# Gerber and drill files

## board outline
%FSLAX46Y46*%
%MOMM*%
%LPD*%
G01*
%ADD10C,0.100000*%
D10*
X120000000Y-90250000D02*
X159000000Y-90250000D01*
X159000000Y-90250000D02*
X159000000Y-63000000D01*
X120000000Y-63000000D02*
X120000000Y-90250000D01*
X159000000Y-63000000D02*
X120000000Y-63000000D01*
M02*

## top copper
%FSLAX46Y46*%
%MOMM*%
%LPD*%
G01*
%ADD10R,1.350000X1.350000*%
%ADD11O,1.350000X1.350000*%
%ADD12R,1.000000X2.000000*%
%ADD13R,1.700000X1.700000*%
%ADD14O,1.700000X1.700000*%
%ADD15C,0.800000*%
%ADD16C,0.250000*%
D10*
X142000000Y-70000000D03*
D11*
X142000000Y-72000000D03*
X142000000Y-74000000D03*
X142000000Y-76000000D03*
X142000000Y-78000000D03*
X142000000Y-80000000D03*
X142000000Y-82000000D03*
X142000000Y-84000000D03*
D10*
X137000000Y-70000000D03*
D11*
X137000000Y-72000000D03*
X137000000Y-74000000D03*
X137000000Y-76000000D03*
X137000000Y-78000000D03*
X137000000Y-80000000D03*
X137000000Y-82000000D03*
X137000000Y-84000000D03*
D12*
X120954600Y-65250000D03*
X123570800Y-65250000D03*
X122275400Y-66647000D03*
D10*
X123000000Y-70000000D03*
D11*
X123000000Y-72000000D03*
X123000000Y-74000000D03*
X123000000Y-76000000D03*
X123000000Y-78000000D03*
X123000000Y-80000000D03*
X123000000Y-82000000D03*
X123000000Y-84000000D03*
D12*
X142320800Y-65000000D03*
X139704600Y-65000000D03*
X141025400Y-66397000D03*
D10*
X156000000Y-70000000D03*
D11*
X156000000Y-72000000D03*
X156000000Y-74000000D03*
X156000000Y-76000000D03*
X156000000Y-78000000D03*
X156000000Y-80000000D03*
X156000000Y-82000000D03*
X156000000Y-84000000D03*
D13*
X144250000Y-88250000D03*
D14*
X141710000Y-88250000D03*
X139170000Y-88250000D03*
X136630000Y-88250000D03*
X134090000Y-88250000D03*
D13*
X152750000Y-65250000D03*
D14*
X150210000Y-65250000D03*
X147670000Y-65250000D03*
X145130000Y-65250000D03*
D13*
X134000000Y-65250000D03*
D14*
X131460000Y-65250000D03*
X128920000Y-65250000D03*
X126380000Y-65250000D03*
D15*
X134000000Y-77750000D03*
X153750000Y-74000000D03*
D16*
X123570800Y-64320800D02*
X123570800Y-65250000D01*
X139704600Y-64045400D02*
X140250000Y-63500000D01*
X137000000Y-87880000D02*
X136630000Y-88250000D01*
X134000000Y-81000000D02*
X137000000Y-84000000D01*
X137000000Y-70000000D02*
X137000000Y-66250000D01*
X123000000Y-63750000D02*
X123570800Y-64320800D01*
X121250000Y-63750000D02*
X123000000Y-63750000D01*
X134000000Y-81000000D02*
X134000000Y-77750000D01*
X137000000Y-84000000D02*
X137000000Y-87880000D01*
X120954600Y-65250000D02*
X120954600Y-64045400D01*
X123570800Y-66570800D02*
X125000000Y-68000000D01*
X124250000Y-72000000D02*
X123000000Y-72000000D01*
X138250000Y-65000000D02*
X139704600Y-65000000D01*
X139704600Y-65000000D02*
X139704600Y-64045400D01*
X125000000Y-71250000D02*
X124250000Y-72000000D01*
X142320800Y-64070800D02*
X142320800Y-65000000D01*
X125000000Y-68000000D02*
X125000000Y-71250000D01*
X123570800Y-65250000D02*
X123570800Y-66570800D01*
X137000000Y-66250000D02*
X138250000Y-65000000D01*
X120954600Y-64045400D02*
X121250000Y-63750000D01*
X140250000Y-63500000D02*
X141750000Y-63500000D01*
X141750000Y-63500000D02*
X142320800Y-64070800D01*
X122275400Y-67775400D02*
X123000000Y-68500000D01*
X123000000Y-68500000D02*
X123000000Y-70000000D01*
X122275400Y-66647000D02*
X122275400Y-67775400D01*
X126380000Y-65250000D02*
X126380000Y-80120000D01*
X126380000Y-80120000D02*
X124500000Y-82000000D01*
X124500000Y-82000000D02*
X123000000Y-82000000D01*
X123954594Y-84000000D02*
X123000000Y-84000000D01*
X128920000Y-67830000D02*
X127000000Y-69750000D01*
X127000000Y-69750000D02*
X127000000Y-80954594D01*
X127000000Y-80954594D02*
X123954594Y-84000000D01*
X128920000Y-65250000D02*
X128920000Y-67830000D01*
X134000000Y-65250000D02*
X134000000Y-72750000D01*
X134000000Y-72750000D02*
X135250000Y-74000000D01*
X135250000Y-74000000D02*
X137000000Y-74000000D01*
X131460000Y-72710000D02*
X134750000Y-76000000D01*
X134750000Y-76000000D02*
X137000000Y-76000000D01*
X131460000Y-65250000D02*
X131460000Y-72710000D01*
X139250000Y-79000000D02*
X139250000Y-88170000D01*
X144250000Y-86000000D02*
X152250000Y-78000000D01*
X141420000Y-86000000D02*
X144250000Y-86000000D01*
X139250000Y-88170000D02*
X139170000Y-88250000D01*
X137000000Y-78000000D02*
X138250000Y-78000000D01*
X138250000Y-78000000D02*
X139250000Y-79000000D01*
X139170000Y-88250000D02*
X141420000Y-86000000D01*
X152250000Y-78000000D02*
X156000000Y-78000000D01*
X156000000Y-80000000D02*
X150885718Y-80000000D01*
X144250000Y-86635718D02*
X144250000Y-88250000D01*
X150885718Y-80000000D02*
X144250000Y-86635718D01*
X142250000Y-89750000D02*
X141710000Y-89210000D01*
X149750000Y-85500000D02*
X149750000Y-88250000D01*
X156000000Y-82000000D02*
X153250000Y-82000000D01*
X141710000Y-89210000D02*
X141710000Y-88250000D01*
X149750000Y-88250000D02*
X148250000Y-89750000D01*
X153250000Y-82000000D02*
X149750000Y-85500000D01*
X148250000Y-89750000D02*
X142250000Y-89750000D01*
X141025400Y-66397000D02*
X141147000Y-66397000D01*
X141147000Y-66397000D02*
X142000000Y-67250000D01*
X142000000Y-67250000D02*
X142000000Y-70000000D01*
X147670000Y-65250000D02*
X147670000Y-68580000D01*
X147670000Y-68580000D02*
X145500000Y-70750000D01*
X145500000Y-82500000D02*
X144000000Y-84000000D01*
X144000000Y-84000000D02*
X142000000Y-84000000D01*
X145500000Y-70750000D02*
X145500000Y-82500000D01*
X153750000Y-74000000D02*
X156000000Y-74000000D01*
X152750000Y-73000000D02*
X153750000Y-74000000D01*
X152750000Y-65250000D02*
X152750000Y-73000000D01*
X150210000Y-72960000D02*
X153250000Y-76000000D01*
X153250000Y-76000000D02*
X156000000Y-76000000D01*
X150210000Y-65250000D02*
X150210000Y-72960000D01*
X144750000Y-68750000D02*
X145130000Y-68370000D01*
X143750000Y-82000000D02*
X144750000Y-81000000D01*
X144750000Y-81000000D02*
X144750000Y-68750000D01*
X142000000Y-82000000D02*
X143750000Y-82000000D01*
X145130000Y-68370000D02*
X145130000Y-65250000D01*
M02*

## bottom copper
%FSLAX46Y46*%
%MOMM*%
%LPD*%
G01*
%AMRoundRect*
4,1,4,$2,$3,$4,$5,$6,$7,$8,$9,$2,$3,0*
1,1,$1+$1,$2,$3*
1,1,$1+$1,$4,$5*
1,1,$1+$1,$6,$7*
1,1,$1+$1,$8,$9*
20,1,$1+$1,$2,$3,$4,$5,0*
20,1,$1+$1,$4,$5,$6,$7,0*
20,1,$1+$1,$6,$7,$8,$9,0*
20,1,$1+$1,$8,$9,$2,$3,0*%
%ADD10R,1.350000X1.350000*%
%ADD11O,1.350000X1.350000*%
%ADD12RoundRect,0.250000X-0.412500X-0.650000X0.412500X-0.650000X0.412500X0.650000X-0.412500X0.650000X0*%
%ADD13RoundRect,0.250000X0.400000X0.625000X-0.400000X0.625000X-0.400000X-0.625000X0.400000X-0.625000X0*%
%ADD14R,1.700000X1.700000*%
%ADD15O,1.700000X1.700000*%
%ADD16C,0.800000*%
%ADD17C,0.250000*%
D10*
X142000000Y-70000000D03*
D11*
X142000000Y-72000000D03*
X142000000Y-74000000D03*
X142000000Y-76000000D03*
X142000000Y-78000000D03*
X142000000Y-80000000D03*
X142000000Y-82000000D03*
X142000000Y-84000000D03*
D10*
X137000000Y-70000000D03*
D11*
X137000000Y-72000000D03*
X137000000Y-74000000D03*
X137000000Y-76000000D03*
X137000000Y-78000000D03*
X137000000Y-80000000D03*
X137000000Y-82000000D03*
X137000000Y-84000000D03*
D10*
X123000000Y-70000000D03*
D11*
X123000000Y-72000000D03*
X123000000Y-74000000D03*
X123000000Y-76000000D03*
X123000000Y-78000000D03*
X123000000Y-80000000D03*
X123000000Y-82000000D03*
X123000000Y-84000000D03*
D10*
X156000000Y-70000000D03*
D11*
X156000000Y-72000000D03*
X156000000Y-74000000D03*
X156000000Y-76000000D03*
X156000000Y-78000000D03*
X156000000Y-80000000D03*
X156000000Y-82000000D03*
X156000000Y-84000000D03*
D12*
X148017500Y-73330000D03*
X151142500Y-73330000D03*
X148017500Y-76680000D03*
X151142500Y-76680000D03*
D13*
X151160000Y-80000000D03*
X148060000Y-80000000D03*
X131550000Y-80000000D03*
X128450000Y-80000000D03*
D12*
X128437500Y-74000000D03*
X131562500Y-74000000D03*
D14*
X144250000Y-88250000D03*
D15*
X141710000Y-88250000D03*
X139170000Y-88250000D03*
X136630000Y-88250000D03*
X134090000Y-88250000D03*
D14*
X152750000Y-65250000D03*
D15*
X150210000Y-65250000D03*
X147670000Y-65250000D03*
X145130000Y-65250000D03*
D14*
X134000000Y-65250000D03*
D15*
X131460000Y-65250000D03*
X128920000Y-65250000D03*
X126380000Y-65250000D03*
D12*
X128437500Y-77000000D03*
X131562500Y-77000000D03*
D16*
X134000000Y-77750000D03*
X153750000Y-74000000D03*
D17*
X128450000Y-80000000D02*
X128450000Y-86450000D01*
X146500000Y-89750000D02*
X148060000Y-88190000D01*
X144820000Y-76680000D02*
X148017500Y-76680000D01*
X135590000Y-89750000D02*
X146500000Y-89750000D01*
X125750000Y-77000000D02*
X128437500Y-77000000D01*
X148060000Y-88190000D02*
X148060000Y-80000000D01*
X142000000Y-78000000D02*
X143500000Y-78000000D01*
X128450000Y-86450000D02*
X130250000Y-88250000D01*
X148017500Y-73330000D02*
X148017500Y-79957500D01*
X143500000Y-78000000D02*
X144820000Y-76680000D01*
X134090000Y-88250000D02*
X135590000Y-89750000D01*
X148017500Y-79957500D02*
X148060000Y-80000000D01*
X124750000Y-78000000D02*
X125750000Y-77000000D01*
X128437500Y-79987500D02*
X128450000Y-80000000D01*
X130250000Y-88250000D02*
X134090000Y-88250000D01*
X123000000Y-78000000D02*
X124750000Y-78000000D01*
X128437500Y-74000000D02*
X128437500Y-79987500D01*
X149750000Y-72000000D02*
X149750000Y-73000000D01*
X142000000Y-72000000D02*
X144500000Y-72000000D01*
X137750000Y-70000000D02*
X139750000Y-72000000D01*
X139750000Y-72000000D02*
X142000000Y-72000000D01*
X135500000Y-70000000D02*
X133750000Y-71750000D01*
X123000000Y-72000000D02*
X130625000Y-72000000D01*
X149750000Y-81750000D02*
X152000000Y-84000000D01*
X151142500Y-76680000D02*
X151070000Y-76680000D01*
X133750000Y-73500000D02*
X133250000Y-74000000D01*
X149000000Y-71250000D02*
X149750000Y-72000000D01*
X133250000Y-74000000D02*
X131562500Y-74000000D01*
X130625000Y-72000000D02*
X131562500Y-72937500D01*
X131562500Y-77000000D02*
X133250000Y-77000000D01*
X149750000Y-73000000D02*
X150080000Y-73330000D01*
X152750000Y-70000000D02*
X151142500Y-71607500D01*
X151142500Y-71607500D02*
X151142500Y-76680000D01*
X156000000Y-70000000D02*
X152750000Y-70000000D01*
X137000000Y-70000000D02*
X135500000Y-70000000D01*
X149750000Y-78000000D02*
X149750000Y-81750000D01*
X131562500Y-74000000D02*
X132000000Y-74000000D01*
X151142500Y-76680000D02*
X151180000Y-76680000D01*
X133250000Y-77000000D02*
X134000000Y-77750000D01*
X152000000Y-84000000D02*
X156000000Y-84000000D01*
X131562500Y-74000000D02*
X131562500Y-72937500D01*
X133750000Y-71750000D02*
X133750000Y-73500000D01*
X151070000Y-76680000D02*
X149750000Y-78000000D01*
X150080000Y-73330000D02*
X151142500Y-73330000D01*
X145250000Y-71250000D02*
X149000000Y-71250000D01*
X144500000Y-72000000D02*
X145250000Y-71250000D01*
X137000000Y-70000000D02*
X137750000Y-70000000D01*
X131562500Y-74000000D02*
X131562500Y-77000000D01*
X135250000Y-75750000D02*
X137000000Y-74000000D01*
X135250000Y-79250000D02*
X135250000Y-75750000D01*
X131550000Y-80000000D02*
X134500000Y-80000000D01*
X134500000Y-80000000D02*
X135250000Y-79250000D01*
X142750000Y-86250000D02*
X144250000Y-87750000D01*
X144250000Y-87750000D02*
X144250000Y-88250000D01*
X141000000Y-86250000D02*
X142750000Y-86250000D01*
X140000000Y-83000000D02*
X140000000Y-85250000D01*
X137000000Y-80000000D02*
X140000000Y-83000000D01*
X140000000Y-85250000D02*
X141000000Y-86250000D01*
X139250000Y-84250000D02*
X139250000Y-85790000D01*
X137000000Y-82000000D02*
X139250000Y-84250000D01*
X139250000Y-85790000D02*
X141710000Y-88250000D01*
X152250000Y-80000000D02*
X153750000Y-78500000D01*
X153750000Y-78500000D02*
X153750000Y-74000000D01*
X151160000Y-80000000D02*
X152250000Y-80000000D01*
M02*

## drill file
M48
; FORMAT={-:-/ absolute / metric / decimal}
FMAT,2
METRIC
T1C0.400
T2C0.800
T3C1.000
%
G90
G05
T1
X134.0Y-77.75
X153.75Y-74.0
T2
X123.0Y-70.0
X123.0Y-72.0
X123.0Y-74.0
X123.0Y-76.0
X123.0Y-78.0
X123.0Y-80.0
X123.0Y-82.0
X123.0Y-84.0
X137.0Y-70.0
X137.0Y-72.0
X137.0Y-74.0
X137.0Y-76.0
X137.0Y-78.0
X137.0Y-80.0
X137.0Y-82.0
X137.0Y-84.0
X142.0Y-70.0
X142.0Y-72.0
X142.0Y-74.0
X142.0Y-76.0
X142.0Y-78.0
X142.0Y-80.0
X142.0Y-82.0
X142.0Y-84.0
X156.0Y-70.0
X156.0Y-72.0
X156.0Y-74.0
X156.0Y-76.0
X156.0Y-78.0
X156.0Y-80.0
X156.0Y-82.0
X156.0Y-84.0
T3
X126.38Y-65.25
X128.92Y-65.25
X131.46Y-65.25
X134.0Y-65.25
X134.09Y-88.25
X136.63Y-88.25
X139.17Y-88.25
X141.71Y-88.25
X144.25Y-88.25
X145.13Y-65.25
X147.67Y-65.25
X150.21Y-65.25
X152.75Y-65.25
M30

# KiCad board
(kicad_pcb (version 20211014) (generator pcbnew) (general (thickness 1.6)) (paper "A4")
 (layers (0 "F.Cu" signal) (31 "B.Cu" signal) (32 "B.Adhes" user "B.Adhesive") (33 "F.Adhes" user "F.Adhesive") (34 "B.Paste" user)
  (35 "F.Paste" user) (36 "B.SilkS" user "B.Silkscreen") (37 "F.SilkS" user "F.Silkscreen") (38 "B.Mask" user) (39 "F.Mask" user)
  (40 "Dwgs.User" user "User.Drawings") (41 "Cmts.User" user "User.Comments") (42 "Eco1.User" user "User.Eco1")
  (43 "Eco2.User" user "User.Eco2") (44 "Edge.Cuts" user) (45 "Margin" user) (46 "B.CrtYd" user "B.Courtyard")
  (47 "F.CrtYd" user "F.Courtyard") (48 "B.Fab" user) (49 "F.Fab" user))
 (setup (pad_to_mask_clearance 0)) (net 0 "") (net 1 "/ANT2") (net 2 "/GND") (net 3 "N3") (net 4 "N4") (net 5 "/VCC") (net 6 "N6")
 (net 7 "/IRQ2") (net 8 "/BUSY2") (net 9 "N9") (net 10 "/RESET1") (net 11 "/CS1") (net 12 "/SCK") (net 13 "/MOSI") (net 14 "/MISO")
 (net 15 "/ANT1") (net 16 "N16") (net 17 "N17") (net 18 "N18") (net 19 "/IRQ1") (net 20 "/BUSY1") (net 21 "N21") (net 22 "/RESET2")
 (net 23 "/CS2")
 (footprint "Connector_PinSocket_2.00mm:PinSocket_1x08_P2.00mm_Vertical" (layer "F.Cu") (at 142 70)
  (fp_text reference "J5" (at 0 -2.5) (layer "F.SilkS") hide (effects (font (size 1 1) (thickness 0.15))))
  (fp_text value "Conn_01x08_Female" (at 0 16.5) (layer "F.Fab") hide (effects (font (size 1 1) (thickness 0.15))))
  (pad "1" thru_hole rect (at 0 0) (size 1.35 1.35) (drill 0.8) (layers *.Cu *.Mask) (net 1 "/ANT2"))
  (pad "2" thru_hole oval (at 0 2) (size 1.35 1.35) (drill 0.8) (layers *.Cu *.Mask) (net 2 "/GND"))
  (pad "3" thru_hole oval (at 0 4) (size 1.35 1.35) (drill 0.8) (layers *.Cu *.Mask) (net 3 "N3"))
  (pad "4" thru_hole oval (at 0 6) (size 1.35 1.35) (drill 0.8) (layers *.Cu *.Mask) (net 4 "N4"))
  (pad "5" thru_hole oval (at 0 8) (size 1.35 1.35) (drill 0.8) (layers *.Cu *.Mask) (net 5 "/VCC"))
  (pad "6" thru_hole oval (at 0 10) (size 1.35 1.35) (drill 0.8) (layers *.Cu *.Mask) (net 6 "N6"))
  (pad "7" thru_hole oval (at 0 12) (size 1.35 1.35) (drill 0.8) (layers *.Cu *.Mask) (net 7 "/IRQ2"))
  (pad "8" thru_hole oval (at 0 14) (size 1.35 1.35) (drill 0.8) (layers *.Cu *.Mask) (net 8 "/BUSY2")))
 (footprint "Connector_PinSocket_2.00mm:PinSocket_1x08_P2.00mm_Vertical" (layer "F.Cu") (at 137 70)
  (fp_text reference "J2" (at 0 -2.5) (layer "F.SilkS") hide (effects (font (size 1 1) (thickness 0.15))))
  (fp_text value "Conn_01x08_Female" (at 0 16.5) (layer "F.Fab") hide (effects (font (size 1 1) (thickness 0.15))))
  (pad "1" thru_hole rect (at 0 0) (size 1.35 1.35) (drill 0.8) (layers *.Cu *.Mask) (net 2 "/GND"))
  (pad "2" thru_hole oval (at 0 2) (size 1.35 1.35) (drill 0.8) (layers *.Cu *.Mask) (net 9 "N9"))
  (pad "3" thru_hole oval (at 0 4) (size 1.35 1.35) (drill 0.8) (layers *.Cu *.Mask) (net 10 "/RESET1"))
  (pad "4" thru_hole oval (at 0 6) (size 1.35 1.35) (drill 0.8) (layers *.Cu *.Mask) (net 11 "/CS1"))
  (pad "5" thru_hole oval (at 0 8) (size 1.35 1.35) (drill 0.8) (layers *.Cu *.Mask) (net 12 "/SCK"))
  (pad "6" thru_hole oval (at 0 10) (size 1.35 1.35) (drill 0.8) (layers *.Cu *.Mask) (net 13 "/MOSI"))
  (pad "7" thru_hole oval (at 0 12) (size 1.35 1.35) (drill 0.8) (layers *.Cu *.Mask) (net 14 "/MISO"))
  (pad "8" thru_hole oval (at 0 14) (size 1.35 1.35) (drill 0.8) (layers *.Cu *.Mask) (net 2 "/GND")))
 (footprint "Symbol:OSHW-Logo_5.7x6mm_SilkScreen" (layer "F.Cu") (at 150.25 86.5)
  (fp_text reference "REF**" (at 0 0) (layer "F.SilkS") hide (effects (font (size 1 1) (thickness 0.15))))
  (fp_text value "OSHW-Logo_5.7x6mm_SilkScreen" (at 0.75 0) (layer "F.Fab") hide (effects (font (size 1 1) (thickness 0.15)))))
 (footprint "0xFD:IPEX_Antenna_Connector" (layer "F.Cu") (at 122.25 65.25 180)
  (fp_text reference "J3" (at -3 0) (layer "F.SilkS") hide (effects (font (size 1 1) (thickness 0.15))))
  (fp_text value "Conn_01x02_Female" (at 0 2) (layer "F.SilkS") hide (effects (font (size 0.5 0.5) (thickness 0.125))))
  (pad "1" smd rect locked (at 1.2954 0 180) (size 1 2) (layers "F.Cu" "F.Paste" "F.Mask") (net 2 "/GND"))
  (pad "1" smd rect locked (at -1.3208 0 90) (size 2 1) (layers "F.Cu" "F.Paste" "F.Mask") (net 2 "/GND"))
  (pad "2" smd rect locked (at -0.0254 -1.397 90) (size 2 1) (layers "F.Cu" "F.Paste" "F.Mask") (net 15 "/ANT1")))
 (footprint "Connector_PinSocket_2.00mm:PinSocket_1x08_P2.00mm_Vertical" (layer "F.Cu") (at 123 70)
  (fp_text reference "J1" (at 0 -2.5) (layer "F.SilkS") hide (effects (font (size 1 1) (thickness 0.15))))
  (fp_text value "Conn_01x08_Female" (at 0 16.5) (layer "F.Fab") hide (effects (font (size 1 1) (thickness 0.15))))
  (pad "1" thru_hole rect (at 0 0) (size 1.35 1.35) (drill 0.8) (layers *.Cu *.Mask) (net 15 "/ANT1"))
  (pad "2" thru_hole oval (at 0 2) (size 1.35 1.35) (drill 0.8) (layers *.Cu *.Mask) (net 2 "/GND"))
  (pad "3" thru_hole oval (at 0 4) (size 1.35 1.35) (drill 0.8) (layers *.Cu *.Mask) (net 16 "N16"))
  (pad "4" thru_hole oval (at 0 6) (size 1.35 1.35) (drill 0.8) (layers *.Cu *.Mask) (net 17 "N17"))
  (pad "5" thru_hole oval (at 0 8) (size 1.35 1.35) (drill 0.8) (layers *.Cu *.Mask) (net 5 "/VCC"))
  (pad "6" thru_hole oval (at 0 10) (size 1.35 1.35) (drill 0.8) (layers *.Cu *.Mask) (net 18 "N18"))
  (pad "7" thru_hole oval (at 0 12) (size 1.35 1.35) (drill 0.8) (layers *.Cu *.Mask) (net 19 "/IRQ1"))
  (pad "8" thru_hole oval (at 0 14) (size 1.35 1.35) (drill 0.8) (layers *.Cu *.Mask) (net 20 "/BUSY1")))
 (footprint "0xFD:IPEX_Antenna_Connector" (layer "F.Cu") (at 141 65 180)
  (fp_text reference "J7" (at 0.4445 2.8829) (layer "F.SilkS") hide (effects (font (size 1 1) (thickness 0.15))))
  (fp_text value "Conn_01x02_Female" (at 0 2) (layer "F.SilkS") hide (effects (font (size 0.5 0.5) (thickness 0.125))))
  (pad "1" smd rect locked (at -1.3208 0 90) (size 2 1) (layers "F.Cu" "F.Paste" "F.Mask") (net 2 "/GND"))
  (pad "1" smd rect locked (at 1.2954 0 180) (size 1 2) (layers "F.Cu" "F.Paste" "F.Mask") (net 2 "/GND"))
  (pad "2" smd rect locked (at -0.0254 -1.397 90) (size 2 1) (layers "F.Cu" "F.Paste" "F.Mask") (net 1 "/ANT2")))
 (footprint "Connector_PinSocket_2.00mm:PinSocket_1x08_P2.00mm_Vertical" (layer "F.Cu") (at 156 70)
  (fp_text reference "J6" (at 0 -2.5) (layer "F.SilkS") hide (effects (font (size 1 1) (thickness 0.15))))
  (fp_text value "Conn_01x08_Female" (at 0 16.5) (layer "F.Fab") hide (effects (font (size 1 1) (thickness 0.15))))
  (pad "1" thru_hole rect (at 0 0) (size 1.35 1.35) (drill 0.8) (layers *.Cu *.Mask) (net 2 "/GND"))
  (pad "2" thru_hole oval (at 0 2) (size 1.35 1.35) (drill 0.8) (layers *.Cu *.Mask) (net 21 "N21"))
  (pad "3" thru_hole oval (at 0 4) (size 1.35 1.35) (drill 0.8) (layers *.Cu *.Mask) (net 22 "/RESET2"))
  (pad "4" thru_hole oval (at 0 6) (size 1.35 1.35) (drill 0.8) (layers *.Cu *.Mask) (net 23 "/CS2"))
  (pad "5" thru_hole oval (at 0 8) (size 1.35 1.35) (drill 0.8) (layers *.Cu *.Mask) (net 12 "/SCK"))
  (pad "6" thru_hole oval (at 0 10) (size 1.35 1.35) (drill 0.8) (layers *.Cu *.Mask) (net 13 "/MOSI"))
  (pad "7" thru_hole oval (at 0 12) (size 1.35 1.35) (drill 0.8) (layers *.Cu *.Mask) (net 14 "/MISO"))
  (pad "8" thru_hole oval (at 0 14) (size 1.35 1.35) (drill 0.8) (layers *.Cu *.Mask) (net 2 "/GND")))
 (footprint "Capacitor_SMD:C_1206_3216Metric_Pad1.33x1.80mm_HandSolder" (layer "B.Cu") (at 149.58 73.33)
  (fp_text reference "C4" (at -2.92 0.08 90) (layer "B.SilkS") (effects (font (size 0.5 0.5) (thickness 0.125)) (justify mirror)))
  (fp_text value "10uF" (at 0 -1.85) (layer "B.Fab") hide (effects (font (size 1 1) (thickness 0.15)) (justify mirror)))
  (pad "1" smd roundrect (at -1.5625 0) (size 1.325 1.8) (layers "B.Cu" "B.Paste" "B.Mask") (roundrect_rratio 0.1886792453) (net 5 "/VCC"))
  (pad "2" smd roundrect (at 1.5625 0) (size 1.325 1.8) (layers "B.Cu" "B.Paste" "B.Mask") (roundrect_rratio 0.1886792453) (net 2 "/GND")))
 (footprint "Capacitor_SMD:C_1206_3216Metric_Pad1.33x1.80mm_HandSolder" (layer "B.Cu") (at 149.58 76.68)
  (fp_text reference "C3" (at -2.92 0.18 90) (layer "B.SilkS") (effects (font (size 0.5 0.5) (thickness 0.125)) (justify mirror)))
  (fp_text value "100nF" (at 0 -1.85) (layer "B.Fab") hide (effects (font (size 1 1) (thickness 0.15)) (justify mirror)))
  (pad "1" smd roundrect (at -1.5625 0) (size 1.325 1.8) (layers "B.Cu" "B.Paste" "B.Mask") (roundrect_rratio 0.1886792453) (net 5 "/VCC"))
  (pad "2" smd roundrect (at 1.5625 0) (size 1.325 1.8) (layers "B.Cu" "B.Paste" "B.Mask") (roundrect_rratio 0.1886792453) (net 2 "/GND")))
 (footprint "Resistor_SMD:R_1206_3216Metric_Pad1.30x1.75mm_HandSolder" (layer "B.Cu") (at 149.61 80 180)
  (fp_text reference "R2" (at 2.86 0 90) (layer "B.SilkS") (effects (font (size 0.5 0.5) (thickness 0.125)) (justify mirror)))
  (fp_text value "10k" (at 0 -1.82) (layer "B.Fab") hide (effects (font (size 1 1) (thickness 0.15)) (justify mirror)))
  (pad "1" smd roundrect (at -1.55 0 180) (size 1.3 1.75) (layers "B.Cu" "B.Paste" "B.Mask") (roundrect_rratio 0.1923076923)
   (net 22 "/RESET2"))
  (pad "2" smd roundrect (at 1.55 0 180) (size 1.3 1.75) (layers "B.Cu" "B.Paste" "B.Mask") (roundrect_rratio 0.1923076923) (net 5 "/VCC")))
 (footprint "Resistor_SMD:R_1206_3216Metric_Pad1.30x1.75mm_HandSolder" (layer "B.Cu") (at 130 80 180)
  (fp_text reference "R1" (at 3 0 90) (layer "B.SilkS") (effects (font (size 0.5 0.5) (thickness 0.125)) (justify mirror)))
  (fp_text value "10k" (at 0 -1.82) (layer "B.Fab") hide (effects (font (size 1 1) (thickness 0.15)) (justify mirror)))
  (pad "1" smd roundrect (at -1.55 0 180) (size 1.3 1.75) (layers "B.Cu" "B.Paste" "B.Mask") (roundrect_rratio 0.1923076923)
   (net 10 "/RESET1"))
  (pad "2" smd roundrect (at 1.55 0 180) (size 1.3 1.75) (layers "B.Cu" "B.Paste" "B.Mask") (roundrect_rratio 0.1923076923) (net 5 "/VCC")))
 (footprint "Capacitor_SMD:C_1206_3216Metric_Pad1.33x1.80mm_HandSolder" (layer "B.Cu") (at 130 74)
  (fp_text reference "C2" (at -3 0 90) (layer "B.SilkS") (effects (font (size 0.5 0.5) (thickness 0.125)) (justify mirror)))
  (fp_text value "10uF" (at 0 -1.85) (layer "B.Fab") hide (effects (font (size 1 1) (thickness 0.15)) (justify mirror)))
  (pad "1" smd roundrect (at -1.5625 0) (size 1.325 1.8) (layers "B.Cu" "B.Paste" "B.Mask") (roundrect_rratio 0.1886792453) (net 5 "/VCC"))
  (pad "2" smd roundrect (at 1.5625 0) (size 1.325 1.8) (layers "B.Cu" "B.Paste" "B.Mask") (roundrect_rratio 0.1886792453) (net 2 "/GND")))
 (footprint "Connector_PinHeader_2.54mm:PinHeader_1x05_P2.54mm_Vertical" (layer "B.Cu") (at 144.25 88.25 90)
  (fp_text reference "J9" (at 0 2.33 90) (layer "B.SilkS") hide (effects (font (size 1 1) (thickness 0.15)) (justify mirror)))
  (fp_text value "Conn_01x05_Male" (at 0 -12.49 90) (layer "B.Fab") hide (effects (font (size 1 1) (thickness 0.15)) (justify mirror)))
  (pad "1" thru_hole rect (at 0 0 90) (size 1.7 1.7) (drill 1) (layers *.Cu *.Mask) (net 13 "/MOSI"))
  (pad "2" thru_hole oval (at 0 -2.54 90) (size 1.7 1.7) (drill 1) (layers *.Cu *.Mask) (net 14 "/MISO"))
  (pad "3" thru_hole oval (at 0 -5.08 90) (size 1.7 1.7) (drill 1) (layers *.Cu *.Mask) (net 12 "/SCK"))
  (pad "4" thru_hole oval (at 0 -7.62 90) (size 1.7 1.7) (drill 1) (layers *.Cu *.Mask) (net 2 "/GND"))
  (pad "5" thru_hole oval (at 0 -10.16 90) (size 1.7 1.7) (drill 1) (layers *.Cu *.Mask) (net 5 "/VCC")))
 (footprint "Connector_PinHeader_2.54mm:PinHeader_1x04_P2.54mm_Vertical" (layer "B.Cu") (at 152.75 65.25 90)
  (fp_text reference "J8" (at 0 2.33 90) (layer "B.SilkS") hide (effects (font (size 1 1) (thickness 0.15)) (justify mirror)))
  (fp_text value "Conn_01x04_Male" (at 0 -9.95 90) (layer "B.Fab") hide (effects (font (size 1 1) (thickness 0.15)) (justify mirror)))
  (pad "1" thru_hole rect (at 0 0 90) (size 1.7 1.7) (drill 1) (layers *.Cu *.Mask) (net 22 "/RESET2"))
  (pad "2" thru_hole oval (at 0 -2.54 90) (size 1.7 1.7) (drill 1) (layers *.Cu *.Mask) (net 23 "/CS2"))
  (pad "3" thru_hole oval (at 0 -5.08 90) (size 1.7 1.7) (drill 1) (layers *.Cu *.Mask) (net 8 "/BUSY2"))
  (pad "4" thru_hole oval (at 0 -7.62 90) (size 1.7 1.7) (drill 1) (layers *.Cu *.Mask) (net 7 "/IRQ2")))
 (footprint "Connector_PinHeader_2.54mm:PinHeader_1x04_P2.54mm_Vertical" (layer "B.Cu") (at 134 65.25 90)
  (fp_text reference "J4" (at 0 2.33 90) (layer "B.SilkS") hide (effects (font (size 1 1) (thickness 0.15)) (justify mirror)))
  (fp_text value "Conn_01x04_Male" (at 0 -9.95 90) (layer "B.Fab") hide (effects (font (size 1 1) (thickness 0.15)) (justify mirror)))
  (pad "1" thru_hole rect (at 0 0 90) (size 1.7 1.7) (drill 1) (layers *.Cu *.Mask) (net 10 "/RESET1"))
  (pad "2" thru_hole oval (at 0 -2.54 90) (size 1.7 1.7) (drill 1) (layers *.Cu *.Mask) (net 11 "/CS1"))
  (pad "3" thru_hole oval (at 0 -5.08 90) (size 1.7 1.7) (drill 1) (layers *.Cu *.Mask) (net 20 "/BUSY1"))
  (pad "4" thru_hole oval (at 0 -7.62 90) (size 1.7 1.7) (drill 1) (layers *.Cu *.Mask) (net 19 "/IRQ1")))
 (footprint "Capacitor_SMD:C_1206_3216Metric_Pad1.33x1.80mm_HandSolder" (layer "B.Cu") (at 130 77)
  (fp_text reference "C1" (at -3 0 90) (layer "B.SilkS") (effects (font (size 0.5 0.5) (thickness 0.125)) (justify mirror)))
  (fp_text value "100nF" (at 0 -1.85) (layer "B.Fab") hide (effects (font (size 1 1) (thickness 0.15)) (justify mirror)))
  (pad "1" smd roundrect (at -1.5625 0) (size 1.325 1.8) (layers "B.Cu" "B.Paste" "B.Mask") (roundrect_rratio 0.1886792453) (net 5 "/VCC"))
  (pad "2" smd roundrect (at 1.5625 0) (size 1.325 1.8) (layers "B.Cu" "B.Paste" "B.Mask") (roundrect_rratio 0.1886792453) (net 2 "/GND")))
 (gr_line (start 120 90.25) (end 159 90.25) (layer "Edge.Cuts") (width 0.1))
 (gr_line (start 159 90.25) (end 159 63) (layer "Edge.Cuts") (width 0.1))
 (gr_line (start 120 63) (end 120 90.25) (layer "Edge.Cuts") (width 0.1))
 (gr_line (start 159 63) (end 120 63) (layer "Edge.Cuts") (width 0.1))
 (segment (start 128.45 80) (end 128.45 86.45) (width 0.25) (layer "B.Cu") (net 5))
 (segment (start 146.5 89.75) (end 148.06 88.19) (width 0.25) (layer "B.Cu") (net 5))
 (segment (start 144.82 76.68) (end 148.0175 76.68) (width 0.25) (layer "B.Cu") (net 5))
 (segment (start 135.59 89.75) (end 146.5 89.75) (width 0.25) (layer "B.Cu") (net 5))
 (segment (start 125.75 77) (end 128.4375 77) (width 0.25) (layer "B.Cu") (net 5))
 (segment (start 148.06 88.19) (end 148.06 80) (width 0.25) (layer "B.Cu") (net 5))
 (segment (start 142 78) (end 143.5 78) (width 0.25) (layer "B.Cu") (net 5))
 (segment (start 128.45 86.45) (end 130.25 88.25) (width 0.25) (layer "B.Cu") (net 5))
 (segment (start 148.0175 73.33) (end 148.0175 79.9575) (width 0.25) (layer "B.Cu") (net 5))
 (segment (start 143.5 78) (end 144.82 76.68) (width 0.25) (layer "B.Cu") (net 5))
 (segment (start 134.09 88.25) (end 135.59 89.75) (width 0.25) (layer "B.Cu") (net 5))
 (segment (start 148.0175 79.9575) (end 148.06 80) (width 0.25) (layer "B.Cu") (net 5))
 (segment (start 124.75 78) (end 125.75 77) (width 0.25) (layer "B.Cu") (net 5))
 (segment (start 128.4375 79.9875) (end 128.45 80) (width 0.25) (layer "B.Cu") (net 5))
 (segment (start 130.25 88.25) (end 134.09 88.25) (width 0.25) (layer "B.Cu") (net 5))
 (segment (start 123 78) (end 124.75 78) (width 0.25) (layer "B.Cu") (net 5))
 (segment (start 128.4375 74) (end 128.4375 79.9875) (width 0.25) (layer "B.Cu") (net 5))
 (segment (start 123.5708 64.3208) (end 123.5708 65.25) (width 0.25) (layer "F.Cu") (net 2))
 (segment (start 139.7046 64.0454) (end 140.25 63.5) (width 0.25) (layer "F.Cu") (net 2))
 (segment (start 137 87.88) (end 136.63 88.25) (width 0.25) (layer "F.Cu") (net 2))
 (segment (start 134 81) (end 137 84) (width 0.25) (layer "F.Cu") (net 2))
 (segment (start 137 70) (end 137 66.25) (width 0.25) (layer "F.Cu") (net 2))
 (segment (start 123 63.75) (end 123.5708 64.3208) (width 0.25) (layer "F.Cu") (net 2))
 (segment (start 121.25 63.75) (end 123 63.75) (width 0.25) (layer "F.Cu") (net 2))
 (segment (start 134 81) (end 134 77.75) (width 0.25) (layer "F.Cu") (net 2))
 (segment (start 137 84) (end 137 87.88) (width 0.25) (layer "F.Cu") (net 2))
 (segment (start 120.9546 65.25) (end 120.9546 64.0454) (width 0.25) (layer "F.Cu") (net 2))
 (segment (start 123.5708 66.5708) (end 125 68) (width 0.25) (layer "F.Cu") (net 2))
 (segment (start 124.25 72) (end 123 72) (width 0.25) (layer "F.Cu") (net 2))
 (segment (start 138.25 65) (end 139.7046 65) (width 0.25) (layer "F.Cu") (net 2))
 (segment (start 139.7046 65) (end 139.7046 64.0454) (width 0.25) (layer "F.Cu") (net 2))
 (segment (start 125 71.25) (end 124.25 72) (width 0.25) (layer "F.Cu") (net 2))
 (segment (start 142.3208 64.0708) (end 142.3208 65) (width 0.25) (layer "F.Cu") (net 2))
 (segment (start 125 68) (end 125 71.25) (width 0.25) (layer "F.Cu") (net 2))
 (segment (start 123.5708 65.25) (end 123.5708 66.5708) (width 0.25) (layer "F.Cu") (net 2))
 (segment (start 137 66.25) (end 138.25 65) (width 0.25) (layer "F.Cu") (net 2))
 (segment (start 120.9546 64.0454) (end 121.25 63.75) (width 0.25) (layer "F.Cu") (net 2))
 (segment (start 140.25 63.5) (end 141.75 63.5) (width 0.25) (layer "F.Cu") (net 2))
 (segment (start 141.75 63.5) (end 142.3208 64.0708) (width 0.25) (layer "F.Cu") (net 2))
 (via (at 134 77.75) (size 0.8) (drill 0.4) (layers "F.Cu" "B.Cu") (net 2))
 (segment (start 149.75 72) (end 149.75 73) (width 0.25) (layer "B.Cu") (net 2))
 (segment (start 142 72) (end 144.5 72) (width 0.25) (layer "B.Cu") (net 2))
 (segment (start 137.75 70) (end 139.75 72) (width 0.25) (layer "B.Cu") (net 2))
 (segment (start 139.75 72) (end 142 72) (width 0.25) (layer "B.Cu") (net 2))
 (segment (start 135.5 70) (end 133.75 71.75) (width 0.25) (layer "B.Cu") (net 2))
 (segment (start 123 72) (end 130.625 72) (width 0.25) (layer "B.Cu") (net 2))
 (segment (start 149.75 81.75) (end 152 84) (width 0.25) (layer "B.Cu") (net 2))
 (segment (start 151.1425 76.68) (end 151.07 76.68) (width 0.25) (layer "B.Cu") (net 2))
 (segment (start 133.75 73.5) (end 133.25 74) (width 0.25) (layer "B.Cu") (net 2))
 (segment (start 149 71.25) (end 149.75 72) (width 0.25) (layer "B.Cu") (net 2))
 (segment (start 133.25 74) (end 131.5625 74) (width 0.25) (layer "B.Cu") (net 2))
 (segment (start 130.625 72) (end 131.5625 72.9375) (width 0.25) (layer "B.Cu") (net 2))
 (segment (start 131.5625 77) (end 133.25 77) (width 0.25) (layer "B.Cu") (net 2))
 (segment (start 149.75 73) (end 150.08 73.33) (width 0.25) (layer "B.Cu") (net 2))
 (segment (start 152.75 70) (end 151.1425 71.6075) (width 0.25) (layer "B.Cu") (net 2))
 (segment (start 151.1425 71.6075) (end 151.1425 76.68) (width 0.25) (layer "B.Cu") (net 2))
 (segment (start 156 70) (end 152.75 70) (width 0.25) (layer "B.Cu") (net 2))
 (segment (start 137 70) (end 135.5 70) (width 0.25) (layer "B.Cu") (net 2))
 (segment (start 149.75 78) (end 149.75 81.75) (width 0.25) (layer "B.Cu") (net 2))
 (segment (start 131.5625 74) (end 132 74) (width 0.25) (layer "B.Cu") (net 2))
 (segment (start 151.1425 76.68) (end 151.18 76.68) (width 0.25) (layer "B.Cu") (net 2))
 (segment (start 133.25 77) (end 134 77.75) (width 0.25) (layer "B.Cu") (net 2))
 (segment (start 152 84) (end 156 84) (width 0.25) (layer "B.Cu") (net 2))
 (segment (start 131.5625 74) (end 131.5625 72.9375) (width 0.25) (layer "B.Cu") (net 2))
 (segment (start 133.75 71.75) (end 133.75 73.5) (width 0.25) (layer "B.Cu") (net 2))
 (segment (start 151.07 76.68) (end 149.75 78) (width 0.25) (layer "B.Cu") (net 2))
 (segment (start 150.08 73.33) (end 151.1425 73.33) (width 0.25) (layer "B.Cu") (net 2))
 (segment (start 145.25 71.25) (end 149 71.25) (width 0.25) (layer "B.Cu") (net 2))
 (segment (start 144.5 72) (end 145.25 71.25) (width 0.25) (layer "B.Cu") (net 2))
 (segment (start 137 70) (end 137.75 70) (width 0.25) (layer "B.Cu") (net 2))
 (segment (start 131.5625 74) (end 131.5625 77) (width 0.25) (layer "B.Cu") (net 2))
 (segment (start 122.2754 67.7754) (end 123 68.5) (width 0.25) (layer "F.Cu") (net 15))
 (segment (start 123 68.5) (end 123 70) (width 0.25) (layer "F.Cu") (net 15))
 (segment (start 122.2754 66.647) (end 122.2754 67.7754) (width 0.25) (layer "F.Cu") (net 15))
 (segment (start 126.38 65.25) (end 126.38 80.12) (width 0.25) (layer "F.Cu") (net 19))
 (segment (start 126.38 80.12) (end 124.5 82) (width 0.25) (layer "F.Cu") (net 19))
 (segment (start 124.5 82) (end 123 82) (width 0.25) (layer "F.Cu") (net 19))
 (segment (start 123.954594 84) (end 123 84) (width 0.25) (layer "F.Cu") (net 20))
 (segment (start 128.92 67.83) (end 127 69.75) (width 0.25) (layer "F.Cu") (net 20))
 (segment (start 127 69.75) (end 127 80.954594) (width 0.25) (layer "F.Cu") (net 20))
 (segment (start 127 80.954594) (end 123.954594 84) (width 0.25) (layer "F.Cu") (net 20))
 (segment (start 128.92 65.25) (end 128.92 67.83) (width 0.25) (layer "F.Cu") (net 20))
 (segment (start 134 65.25) (end 134 72.75) (width 0.25) (layer "F.Cu") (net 10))
 (segment (start 134 72.75) (end 135.25 74) (width 0.25) (layer "F.Cu") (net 10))
 (segment (start 135.25 74) (end 137 74) (width 0.25) (layer "F.Cu") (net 10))
 (segment (start 135.25 75.75) (end 137 74) (width 0.25) (layer "B.Cu") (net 10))
 (segment (start 135.25 79.25) (end 135.25 75.75) (width 0.25) (layer "B.Cu") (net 10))
 (segment (start 131.55 80) (end 134.5 80) (width 0.25) (layer "B.Cu") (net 10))
 (segment (start 134.5 80) (end 135.25 79.25) (width 0.25) (layer "B.Cu") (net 10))
 (segment (start 131.46 72.71) (end 134.75 76) (width 0.25) (layer "F.Cu") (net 11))
 (segment (start 134.75 76) (end 137 76) (width 0.25) (layer "F.Cu") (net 11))
 (segment (start 131.46 65.25) (end 131.46 72.71) (width 0.25) (layer "F.Cu") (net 11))
 (segment (start 139.25 79) (end 139.25 88.17) (width 0.25) (layer "F.Cu") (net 12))
 (segment (start 144.25 86) (end 152.25 78) (width 0.25) (layer "F.Cu") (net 12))
 (segment (start 141.42 86) (end 144.25 86) (width 0.25) (layer "F.Cu") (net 12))
 (segment (start 139.25 88.17) (end 139.17 88.25) (width 0.25) (layer "F.Cu") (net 12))
 (segment (start 137 78) (end 138.25 78) (width 0.25) (layer "F.Cu") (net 12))
 (segment (start 138.25 78) (end 139.25 79) (width 0.25) (layer "F.Cu") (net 12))
 (segment (start 139.17 88.25) (end 141.42 86) (width 0.25) (layer "F.Cu") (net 12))
 (segment (start 152.25 78) (end 156 78) (width 0.25) (layer "F.Cu") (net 12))
 (segment (start 156 80) (end 150.885718 80) (width 0.25) (layer "F.Cu") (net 13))
 (segment (start 144.25 86.635718) (end 144.25 88.25) (width 0.25) (layer "F.Cu") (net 13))
 (segment (start 150.885718 80) (end 144.25 86.635718) (width 0.25) (layer "F.Cu") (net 13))
 (segment (start 142.75 86.25) (end 144.25 87.75) (width 0.25) (layer "B.Cu") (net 13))
 (segment (start 144.25 87.75) (end 144.25 88.25) (width 0.25) (layer "B.Cu") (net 13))
 (segment (start 141 86.25) (end 142.75 86.25) (width 0.25) (layer "B.Cu") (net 13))
 (segment (start 140 83) (end 140 85.25) (width 0.25) (layer "B.Cu") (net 13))
 (segment (start 137 80) (end 140 83) (width 0.25) (layer "B.Cu") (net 13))
 (segment (start 140 85.25) (end 141 86.25) (width 0.25) (layer "B.Cu") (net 13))
 (segment (start 142.25 89.75) (end 141.71 89.21) (width 0.25) (layer "F.Cu") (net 14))
 (segment (start 149.75 85.5) (end 149.75 88.25) (width 0.25) (layer "F.Cu") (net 14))
 (segment (start 156 82) (end 153.25 82) (width 0.25) (layer "F.Cu") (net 14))
 (segment (start 141.71 89.21) (end 141.71 88.25) (width 0.25) (layer "F.Cu") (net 14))
 (segment (start 149.75 88.25) (end 148.25 89.75) (width 0.25) (layer "F.Cu") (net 14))
 (segment (start 153.25 82) (end 149.75 85.5) (width 0.25) (layer "F.Cu") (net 14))
 (segment (start 148.25 89.75) (end 142.25 89.75) (width 0.25) (layer "F.Cu") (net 14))
 (segment (start 139.25 84.25) (end 139.25 85.79) (width 0.25) (layer "B.Cu") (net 14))
 (segment (start 137 82) (end 139.25 84.25) (width 0.25) (layer "B.Cu") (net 14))
 (segment (start 139.25 85.79) (end 141.71 88.25) (width 0.25) (layer "B.Cu") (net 14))
 (segment (start 141.0254 66.397) (end 141.147 66.397) (width 0.25) (layer "F.Cu") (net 1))
 (segment (start 141.147 66.397) (end 142 67.25) (width 0.25) (layer "F.Cu") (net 1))
 (segment (start 142 67.25) (end 142 70) (width 0.25) (layer "F.Cu") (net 1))
 (segment (start 147.67 65.25) (end 147.67 68.58) (width 0.25) (layer "F.Cu") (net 8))
 (segment (start 147.67 68.58) (end 145.5 70.75) (width 0.25) (layer "F.Cu") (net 8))
 (segment (start 145.5 82.5) (end 144 84) (width 0.25) (layer "F.Cu") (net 8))
 (segment (start 144 84) (end 142 84) (width 0.25) (layer "F.Cu") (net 8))
 (segment (start 145.5 70.75) (end 145.5 82.5) (width 0.25) (layer "F.Cu") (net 8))
 (segment (start 153.75 74) (end 156 74) (width 0.25) (layer "F.Cu") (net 22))
 (segment (start 152.75 73) (end 153.75 74) (width 0.25) (layer "F.Cu") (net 22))
 (segment (start 152.75 65.25) (end 152.75 73) (width 0.25) (layer "F.Cu") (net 22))
 (via (at 153.75 74) (size 0.8) (drill 0.4) (layers "F.Cu" "B.Cu") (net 22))
 (segment (start 152.25 80) (end 153.75 78.5) (width 0.25) (layer "B.Cu") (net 22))
 (segment (start 153.75 78.5) (end 153.75 74) (width 0.25) (layer "B.Cu") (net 22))
 (segment (start 151.16 80) (end 152.25 80) (width 0.25) (layer "B.Cu") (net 22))
 (segment (start 150.21 72.96) (end 153.25 76) (width 0.25) (layer "F.Cu") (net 23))
 (segment (start 153.25 76) (end 156 76) (width 0.25) (layer "F.Cu") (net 23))
 (segment (start 150.21 65.25) (end 150.21 72.96) (width 0.25) (layer "F.Cu") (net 23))
 (segment (start 144.75 68.75) (end 145.13 68.37) (width 0.25) (layer "F.Cu") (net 7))
 (segment (start 143.75 82) (end 144.75 81) (width 0.25) (layer "F.Cu") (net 7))
 (segment (start 144.75 81) (end 144.75 68.75) (width 0.25) (layer "F.Cu") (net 7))
 (segment (start 142 82) (end 143.75 82) (width 0.25) (layer "F.Cu") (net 7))
 (segment (start 145.13 68.37) (end 145.13 65.25) (width 0.25) (layer "F.Cu") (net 7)))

